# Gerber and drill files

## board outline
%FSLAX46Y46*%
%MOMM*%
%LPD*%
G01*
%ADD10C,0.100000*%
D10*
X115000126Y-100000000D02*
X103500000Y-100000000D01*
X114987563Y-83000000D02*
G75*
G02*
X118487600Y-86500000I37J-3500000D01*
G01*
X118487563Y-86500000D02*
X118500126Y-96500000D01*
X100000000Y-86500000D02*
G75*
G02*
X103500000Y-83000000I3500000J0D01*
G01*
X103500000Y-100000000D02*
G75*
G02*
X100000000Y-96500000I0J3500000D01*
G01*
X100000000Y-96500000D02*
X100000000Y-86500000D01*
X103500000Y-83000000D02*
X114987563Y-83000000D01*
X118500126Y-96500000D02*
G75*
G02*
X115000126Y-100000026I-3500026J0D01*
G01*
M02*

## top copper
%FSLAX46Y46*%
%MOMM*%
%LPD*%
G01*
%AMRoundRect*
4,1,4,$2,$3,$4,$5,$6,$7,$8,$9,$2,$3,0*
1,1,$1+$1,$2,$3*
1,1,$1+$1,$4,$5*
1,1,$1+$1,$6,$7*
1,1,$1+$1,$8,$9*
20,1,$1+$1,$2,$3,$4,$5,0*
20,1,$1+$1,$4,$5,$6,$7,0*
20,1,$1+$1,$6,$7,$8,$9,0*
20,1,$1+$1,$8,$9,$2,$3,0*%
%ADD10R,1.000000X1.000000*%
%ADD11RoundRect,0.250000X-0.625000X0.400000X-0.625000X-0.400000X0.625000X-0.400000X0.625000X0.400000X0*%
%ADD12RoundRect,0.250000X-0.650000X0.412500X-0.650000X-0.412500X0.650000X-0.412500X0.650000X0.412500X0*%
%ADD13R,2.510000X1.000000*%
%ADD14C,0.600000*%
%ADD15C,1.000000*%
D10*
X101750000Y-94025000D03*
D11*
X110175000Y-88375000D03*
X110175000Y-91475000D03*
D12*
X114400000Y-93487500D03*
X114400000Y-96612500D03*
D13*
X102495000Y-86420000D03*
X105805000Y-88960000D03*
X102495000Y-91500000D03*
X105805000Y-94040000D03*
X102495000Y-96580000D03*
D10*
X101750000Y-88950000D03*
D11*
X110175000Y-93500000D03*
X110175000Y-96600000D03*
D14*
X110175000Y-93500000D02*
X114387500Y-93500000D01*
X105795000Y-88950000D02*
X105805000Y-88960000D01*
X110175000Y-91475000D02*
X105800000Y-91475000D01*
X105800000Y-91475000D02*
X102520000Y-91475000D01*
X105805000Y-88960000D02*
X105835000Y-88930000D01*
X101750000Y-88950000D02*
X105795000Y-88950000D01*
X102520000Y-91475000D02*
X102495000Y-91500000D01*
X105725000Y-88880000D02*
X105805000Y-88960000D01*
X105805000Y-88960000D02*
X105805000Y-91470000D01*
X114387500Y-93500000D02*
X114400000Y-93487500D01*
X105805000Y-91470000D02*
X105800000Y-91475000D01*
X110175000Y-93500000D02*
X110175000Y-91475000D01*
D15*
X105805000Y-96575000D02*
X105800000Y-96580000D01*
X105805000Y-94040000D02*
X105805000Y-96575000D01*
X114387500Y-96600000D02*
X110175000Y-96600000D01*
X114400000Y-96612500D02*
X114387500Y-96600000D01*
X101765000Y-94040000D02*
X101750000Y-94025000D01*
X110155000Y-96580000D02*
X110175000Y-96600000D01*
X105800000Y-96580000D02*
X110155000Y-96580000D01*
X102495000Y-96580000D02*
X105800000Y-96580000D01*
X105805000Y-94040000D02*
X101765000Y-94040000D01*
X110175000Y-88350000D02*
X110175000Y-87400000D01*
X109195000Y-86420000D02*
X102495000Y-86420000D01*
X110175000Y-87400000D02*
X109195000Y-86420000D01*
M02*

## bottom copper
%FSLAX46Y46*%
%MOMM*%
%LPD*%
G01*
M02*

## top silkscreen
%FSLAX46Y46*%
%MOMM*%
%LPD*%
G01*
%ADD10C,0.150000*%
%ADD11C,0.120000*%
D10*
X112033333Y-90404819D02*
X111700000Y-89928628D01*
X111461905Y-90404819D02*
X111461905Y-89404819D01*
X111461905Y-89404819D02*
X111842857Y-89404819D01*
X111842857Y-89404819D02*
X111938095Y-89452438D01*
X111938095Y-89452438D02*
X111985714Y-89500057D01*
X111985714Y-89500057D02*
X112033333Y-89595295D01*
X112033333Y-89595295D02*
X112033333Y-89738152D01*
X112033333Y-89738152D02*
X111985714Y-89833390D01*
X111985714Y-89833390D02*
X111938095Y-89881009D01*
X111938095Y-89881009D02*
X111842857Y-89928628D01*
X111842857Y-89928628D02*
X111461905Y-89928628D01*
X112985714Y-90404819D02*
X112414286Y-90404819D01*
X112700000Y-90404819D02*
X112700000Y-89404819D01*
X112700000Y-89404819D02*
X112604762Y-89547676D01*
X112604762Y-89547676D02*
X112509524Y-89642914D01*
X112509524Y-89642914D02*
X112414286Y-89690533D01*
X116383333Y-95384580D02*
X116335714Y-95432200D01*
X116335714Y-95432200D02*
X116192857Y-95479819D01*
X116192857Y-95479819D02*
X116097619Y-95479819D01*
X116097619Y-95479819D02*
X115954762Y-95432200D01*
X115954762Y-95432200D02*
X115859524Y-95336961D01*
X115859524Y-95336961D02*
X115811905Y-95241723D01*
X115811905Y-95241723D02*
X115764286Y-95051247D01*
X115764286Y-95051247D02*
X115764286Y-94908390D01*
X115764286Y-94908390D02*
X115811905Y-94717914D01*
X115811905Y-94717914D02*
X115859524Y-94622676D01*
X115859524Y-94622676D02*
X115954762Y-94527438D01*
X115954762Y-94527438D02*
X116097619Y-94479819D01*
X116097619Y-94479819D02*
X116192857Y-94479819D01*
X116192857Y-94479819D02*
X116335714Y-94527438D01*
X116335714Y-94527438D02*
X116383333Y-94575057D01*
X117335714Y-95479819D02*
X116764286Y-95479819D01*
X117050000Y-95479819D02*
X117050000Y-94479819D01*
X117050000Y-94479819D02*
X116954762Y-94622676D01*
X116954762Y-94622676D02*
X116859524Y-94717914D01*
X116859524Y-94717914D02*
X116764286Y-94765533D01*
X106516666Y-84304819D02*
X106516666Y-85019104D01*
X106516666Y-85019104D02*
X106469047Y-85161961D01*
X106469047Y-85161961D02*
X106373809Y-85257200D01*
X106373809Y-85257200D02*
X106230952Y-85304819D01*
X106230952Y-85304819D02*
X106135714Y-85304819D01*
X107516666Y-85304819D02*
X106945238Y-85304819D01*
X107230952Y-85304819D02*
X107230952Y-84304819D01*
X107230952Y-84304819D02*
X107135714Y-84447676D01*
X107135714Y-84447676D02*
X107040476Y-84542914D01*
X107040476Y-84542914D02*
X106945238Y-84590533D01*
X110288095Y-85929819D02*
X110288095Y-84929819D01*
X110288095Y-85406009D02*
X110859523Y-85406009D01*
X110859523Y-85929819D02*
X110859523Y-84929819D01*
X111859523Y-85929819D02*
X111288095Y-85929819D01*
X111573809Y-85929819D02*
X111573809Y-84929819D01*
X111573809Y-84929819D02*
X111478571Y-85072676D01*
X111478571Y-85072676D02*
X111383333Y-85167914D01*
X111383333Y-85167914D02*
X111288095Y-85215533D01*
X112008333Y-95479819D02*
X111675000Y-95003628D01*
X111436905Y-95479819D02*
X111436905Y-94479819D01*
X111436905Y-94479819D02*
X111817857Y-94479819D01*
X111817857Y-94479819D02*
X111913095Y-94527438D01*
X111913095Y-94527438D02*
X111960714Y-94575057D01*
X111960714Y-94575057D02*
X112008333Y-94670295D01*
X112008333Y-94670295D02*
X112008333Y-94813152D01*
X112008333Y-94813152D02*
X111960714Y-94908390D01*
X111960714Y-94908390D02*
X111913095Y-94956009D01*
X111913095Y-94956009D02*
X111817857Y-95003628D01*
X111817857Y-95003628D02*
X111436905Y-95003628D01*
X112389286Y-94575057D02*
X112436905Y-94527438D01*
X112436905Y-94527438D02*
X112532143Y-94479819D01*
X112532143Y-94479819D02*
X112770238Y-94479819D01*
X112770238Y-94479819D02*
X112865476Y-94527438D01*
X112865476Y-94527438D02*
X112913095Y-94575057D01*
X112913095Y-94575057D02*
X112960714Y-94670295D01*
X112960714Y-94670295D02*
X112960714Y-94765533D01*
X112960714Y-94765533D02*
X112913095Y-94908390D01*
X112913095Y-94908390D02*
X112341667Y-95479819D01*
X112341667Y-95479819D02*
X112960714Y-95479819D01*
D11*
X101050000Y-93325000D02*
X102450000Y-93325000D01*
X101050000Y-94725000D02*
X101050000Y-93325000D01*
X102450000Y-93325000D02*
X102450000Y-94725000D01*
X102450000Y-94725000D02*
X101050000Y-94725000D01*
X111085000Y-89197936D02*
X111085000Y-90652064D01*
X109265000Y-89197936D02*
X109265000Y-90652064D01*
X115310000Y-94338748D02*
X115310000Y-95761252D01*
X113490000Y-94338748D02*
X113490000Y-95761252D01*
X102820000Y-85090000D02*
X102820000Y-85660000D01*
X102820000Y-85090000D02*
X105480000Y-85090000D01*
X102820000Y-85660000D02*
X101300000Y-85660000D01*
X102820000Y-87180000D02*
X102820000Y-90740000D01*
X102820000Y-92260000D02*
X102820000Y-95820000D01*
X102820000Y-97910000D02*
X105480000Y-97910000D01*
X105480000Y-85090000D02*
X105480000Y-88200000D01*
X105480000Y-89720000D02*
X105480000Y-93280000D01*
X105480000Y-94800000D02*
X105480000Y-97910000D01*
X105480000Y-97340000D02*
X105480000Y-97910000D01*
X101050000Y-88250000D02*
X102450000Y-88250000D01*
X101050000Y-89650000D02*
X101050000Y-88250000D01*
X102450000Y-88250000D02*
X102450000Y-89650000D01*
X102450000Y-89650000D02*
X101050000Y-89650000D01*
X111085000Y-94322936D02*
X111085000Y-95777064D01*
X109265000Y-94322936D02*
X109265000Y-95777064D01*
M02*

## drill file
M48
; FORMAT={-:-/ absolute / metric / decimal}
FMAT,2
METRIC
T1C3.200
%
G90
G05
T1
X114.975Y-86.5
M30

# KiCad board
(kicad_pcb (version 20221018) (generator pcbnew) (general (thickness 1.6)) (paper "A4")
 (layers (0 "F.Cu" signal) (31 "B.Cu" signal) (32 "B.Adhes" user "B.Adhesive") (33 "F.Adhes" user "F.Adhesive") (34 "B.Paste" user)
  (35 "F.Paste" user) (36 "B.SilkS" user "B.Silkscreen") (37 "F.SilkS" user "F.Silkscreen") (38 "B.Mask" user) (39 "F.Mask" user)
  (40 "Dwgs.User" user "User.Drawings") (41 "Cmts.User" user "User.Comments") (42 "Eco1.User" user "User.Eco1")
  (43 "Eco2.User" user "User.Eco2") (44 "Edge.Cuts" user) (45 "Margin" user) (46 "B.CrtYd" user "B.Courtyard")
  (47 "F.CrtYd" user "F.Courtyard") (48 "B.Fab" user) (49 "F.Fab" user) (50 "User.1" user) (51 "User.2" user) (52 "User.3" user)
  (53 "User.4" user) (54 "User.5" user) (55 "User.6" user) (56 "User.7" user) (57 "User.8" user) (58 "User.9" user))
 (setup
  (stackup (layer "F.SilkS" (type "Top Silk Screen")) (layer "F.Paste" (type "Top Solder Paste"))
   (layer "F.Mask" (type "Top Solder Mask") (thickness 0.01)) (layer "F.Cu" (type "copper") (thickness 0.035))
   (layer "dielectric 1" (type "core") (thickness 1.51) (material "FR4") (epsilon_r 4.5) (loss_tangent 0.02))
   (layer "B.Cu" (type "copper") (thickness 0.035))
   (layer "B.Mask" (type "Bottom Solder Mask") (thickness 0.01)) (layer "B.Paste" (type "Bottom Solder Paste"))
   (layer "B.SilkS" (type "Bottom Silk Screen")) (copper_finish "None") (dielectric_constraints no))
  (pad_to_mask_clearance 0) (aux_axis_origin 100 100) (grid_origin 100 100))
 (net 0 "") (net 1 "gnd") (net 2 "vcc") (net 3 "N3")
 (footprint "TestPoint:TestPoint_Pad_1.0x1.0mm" (layer "F.Cu") (at 101.75 94.025)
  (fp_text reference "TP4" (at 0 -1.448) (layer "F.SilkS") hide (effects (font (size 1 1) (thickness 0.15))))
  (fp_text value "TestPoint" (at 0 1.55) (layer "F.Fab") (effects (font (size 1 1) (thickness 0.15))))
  (fp_line (start -0.7 -0.7) (end 0.7 -0.7) (stroke (width 0.12) (type solid)) (layer "F.SilkS"))
  (fp_line (start -0.7 0.7) (end -0.7 -0.7) (stroke (width 0.12) (type solid)) (layer "F.SilkS"))
  (fp_line (start 0.7 -0.7) (end 0.7 0.7) (stroke (width 0.12) (type solid)) (layer "F.SilkS"))
  (fp_line (start 0.7 0.7) (end -0.7 0.7) (stroke (width 0.12) (type solid)) (layer "F.SilkS"))
  (pad "1" smd rect (at 0 0) (size 1 1) (layers "F.Cu" "F.Mask") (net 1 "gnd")))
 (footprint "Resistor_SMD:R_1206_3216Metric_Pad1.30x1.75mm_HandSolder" (layer "F.Cu") (at 110.175 89.925 -90)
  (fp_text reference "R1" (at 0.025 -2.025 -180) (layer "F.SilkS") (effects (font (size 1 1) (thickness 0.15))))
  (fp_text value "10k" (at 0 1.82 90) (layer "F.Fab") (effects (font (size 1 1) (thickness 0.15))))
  (fp_line (start -0.727064 -0.91) (end 0.727064 -0.91) (stroke (width 0.12) (type solid)) (layer "F.SilkS"))
  (fp_line (start -0.727064 0.91) (end 0.727064 0.91) (stroke (width 0.12) (type solid)) (layer "F.SilkS"))
  (pad "1" smd roundrect (at -1.55 0 270) (size 1.3 1.75) (layers "F.Cu" "F.Paste" "F.Mask") (roundrect_rratio 0.1923076923) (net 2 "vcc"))
  (pad "2" smd roundrect (at 1.55 0 270) (size 1.3 1.75) (layers "F.Cu" "F.Paste" "F.Mask") (roundrect_rratio 0.1923076923) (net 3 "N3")))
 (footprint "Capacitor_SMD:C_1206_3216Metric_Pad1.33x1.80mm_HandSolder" (layer "F.Cu") (at 114.4 95.05 -90)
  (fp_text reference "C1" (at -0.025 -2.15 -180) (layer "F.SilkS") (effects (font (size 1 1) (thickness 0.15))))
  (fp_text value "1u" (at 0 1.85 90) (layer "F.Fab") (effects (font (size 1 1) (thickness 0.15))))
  (fp_line (start -0.711252 -0.91) (end 0.711252 -0.91) (stroke (width 0.12) (type solid)) (layer "F.SilkS"))
  (fp_line (start -0.711252 0.91) (end 0.711252 0.91) (stroke (width 0.12) (type solid)) (layer "F.SilkS"))
  (pad "1" smd roundrect (at -1.5625 0 270) (size 1.325 1.8) (layers "F.Cu" "F.Paste" "F.Mask") (roundrect_rratio 0.1886792453) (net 3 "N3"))
  (pad "2" smd roundrect (at 1.5625 0 270) (size 1.325 1.8) (layers "F.Cu" "F.Paste" "F.Mask") (roundrect_rratio 0.1886792453) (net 1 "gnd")))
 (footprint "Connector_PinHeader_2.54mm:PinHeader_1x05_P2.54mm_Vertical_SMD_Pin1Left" (layer "F.Cu") (at 104.15 91.5)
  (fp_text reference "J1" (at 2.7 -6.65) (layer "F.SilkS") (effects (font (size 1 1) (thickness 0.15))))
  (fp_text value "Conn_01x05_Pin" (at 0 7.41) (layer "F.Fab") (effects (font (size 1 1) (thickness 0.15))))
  (fp_line (start -1.33 -6.41) (end -1.33 -5.84) (stroke (width 0.12) (type solid)) (layer "F.SilkS"))
  (fp_line (start -1.33 -6.41) (end 1.33 -6.41) (stroke (width 0.12) (type solid)) (layer "F.SilkS"))
  (fp_line (start -1.33 -5.84) (end -2.85 -5.84) (stroke (width 0.12) (type solid)) (layer "F.SilkS"))
  (fp_line (start -1.33 -4.32) (end -1.33 -0.76) (stroke (width 0.12) (type solid)) (layer "F.SilkS"))
  (fp_line (start -1.33 0.76) (end -1.33 4.32) (stroke (width 0.12) (type solid)) (layer "F.SilkS"))
  (fp_line (start -1.33 6.41) (end 1.33 6.41) (stroke (width 0.12) (type solid)) (layer "F.SilkS"))
  (fp_line (start 1.33 -6.41) (end 1.33 -3.3) (stroke (width 0.12) (type solid)) (layer "F.SilkS"))
  (fp_line (start 1.33 -1.78) (end 1.33 1.78) (stroke (width 0.12) (type solid)) (layer "F.SilkS"))
  (fp_line (start 1.33 3.3) (end 1.33 6.41) (stroke (width 0.12) (type solid)) (layer "F.SilkS"))
  (fp_line (start 1.33 5.84) (end 1.33 6.41) (stroke (width 0.12) (type solid)) (layer "F.SilkS"))
  (pad "1" smd rect (at -1.655 -5.08) (size 2.51 1) (layers "F.Cu" "F.Paste" "F.Mask") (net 2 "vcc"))
  (pad "2" smd rect (at 1.655 -2.54) (size 2.51 1) (layers "F.Cu" "F.Paste" "F.Mask") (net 3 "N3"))
  (pad "3" smd rect (at -1.655 0) (size 2.51 1) (layers "F.Cu" "F.Paste" "F.Mask") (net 3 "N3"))
  (pad "4" smd rect (at 1.655 2.54) (size 2.51 1) (layers "F.Cu" "F.Paste" "F.Mask") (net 1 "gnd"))
  (pad "5" smd rect (at -1.655 5.08) (size 2.51 1) (layers "F.Cu" "F.Paste" "F.Mask") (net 1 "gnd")))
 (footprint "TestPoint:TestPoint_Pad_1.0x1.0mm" (layer "F.Cu") (at 101.75 88.95)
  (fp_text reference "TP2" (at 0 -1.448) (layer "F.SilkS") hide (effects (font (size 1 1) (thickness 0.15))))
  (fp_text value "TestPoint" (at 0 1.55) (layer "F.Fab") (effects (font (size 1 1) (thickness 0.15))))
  (fp_line (start -0.7 -0.7) (end 0.7 -0.7) (stroke (width 0.12) (type solid)) (layer "F.SilkS"))
  (fp_line (start -0.7 0.7) (end -0.7 -0.7) (stroke (width 0.12) (type solid)) (layer "F.SilkS"))
  (fp_line (start 0.7 -0.7) (end 0.7 0.7) (stroke (width 0.12) (type solid)) (layer "F.SilkS"))
  (fp_line (start 0.7 0.7) (end -0.7 0.7) (stroke (width 0.12) (type solid)) (layer "F.SilkS"))
  (pad "1" smd rect (at 0 0) (size 1 1) (layers "F.Cu" "F.Mask") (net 3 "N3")))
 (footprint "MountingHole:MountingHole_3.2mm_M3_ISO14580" (layer "F.Cu") (at 114.975 86.5)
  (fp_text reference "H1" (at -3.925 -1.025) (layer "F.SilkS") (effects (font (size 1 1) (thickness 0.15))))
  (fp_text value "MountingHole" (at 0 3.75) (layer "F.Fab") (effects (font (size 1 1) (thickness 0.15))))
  (pad "" np_thru_hole circle (at 0 0) (size 3.2 3.2) (drill 3.2) (layers "*.Cu" "*.Mask")))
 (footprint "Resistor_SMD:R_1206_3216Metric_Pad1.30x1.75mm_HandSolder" (layer "F.Cu") (at 110.175 95.05 -90)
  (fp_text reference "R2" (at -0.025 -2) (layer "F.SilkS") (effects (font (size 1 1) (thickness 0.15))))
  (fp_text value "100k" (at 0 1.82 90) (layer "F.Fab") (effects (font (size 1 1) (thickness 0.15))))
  (fp_line (start -0.727064 -0.91) (end 0.727064 -0.91) (stroke (width 0.12) (type solid)) (layer "F.SilkS"))
  (fp_line (start -0.727064 0.91) (end 0.727064 0.91) (stroke (width 0.12) (type solid)) (layer "F.SilkS"))
  (pad "1" smd roundrect (at -1.55 0 270) (size 1.3 1.75) (layers "F.Cu" "F.Paste" "F.Mask") (roundrect_rratio 0.1923076923) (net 3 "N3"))
  (pad "2" smd roundrect (at 1.55 0 270) (size 1.3 1.75) (layers "F.Cu" "F.Paste" "F.Mask") (roundrect_rratio 0.1923076923) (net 1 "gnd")))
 (gr_line (start 115.000126 100) (end 103.5 100) (stroke (width 0.1) (type default)) (layer "Edge.Cuts"))
 (gr_arc (start 114.987563 83) (mid 117.462436 84.025126) (end 118.487563 86.5) (stroke (width 0.1) (type default)) (layer "Edge.Cuts"))
 (gr_line (start 118.487563 86.5) (end 118.500126 96.5) (stroke (width 0.1) (type default)) (layer "Edge.Cuts"))
 (gr_arc (start 100 86.5) (mid 101.025126 84.025126) (end 103.5 83) (stroke (width 0.1) (type default)) (layer "Edge.Cuts"))
 (gr_arc (start 103.5 100) (mid 101.025126 98.974874) (end 100 96.5) (stroke (width 0.1) (type default)) (layer "Edge.Cuts"))
 (gr_line (start 100 96.5) (end 100 86.5) (stroke (width 0.1) (type default)) (layer "Edge.Cuts"))
 (gr_line (start 103.5 83) (end 114.987563 83) (stroke (width 0.1) (type default)) (layer "Edge.Cuts"))
 (gr_arc (start 118.500126 96.5) (mid 117.475 98.974874) (end 115.000126 100) (stroke (width 0.1) (type default)) (layer "Edge.Cuts"))
 (segment (start 110.175 93.5) (end 114.3875 93.5) (width 0.6) (layer "F.Cu") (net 3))
 (segment (start 105.795 88.95) (end 105.805 88.96) (width 0.6) (layer "F.Cu") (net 3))
 (segment (start 110.175 91.475) (end 105.8 91.475) (width 0.6) (layer "F.Cu") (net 3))
 (segment (start 105.8 91.475) (end 102.52 91.475) (width 0.6) (layer "F.Cu") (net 3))
 (segment (start 105.805 88.96) (end 105.835 88.93) (width 0.6) (layer "F.Cu") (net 3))
 (segment (start 101.75 88.95) (end 105.795 88.95) (width 0.6) (layer "F.Cu") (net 3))
 (segment (start 102.52 91.475) (end 102.495 91.5) (width 0.6) (layer "F.Cu") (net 3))
 (segment (start 105.725 88.88) (end 105.805 88.96) (width 0.6) (layer "F.Cu") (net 3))
 (segment (start 105.805 88.96) (end 105.805 91.47) (width 0.6) (layer "F.Cu") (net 3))
 (segment (start 114.3875 93.5) (end 114.4 93.4875) (width 0.6) (layer "F.Cu") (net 3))
 (segment (start 105.805 91.47) (end 105.8 91.475) (width 0.6) (layer "F.Cu") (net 3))
 (segment (start 110.175 93.5) (end 110.175 91.475) (width 0.6) (layer "F.Cu") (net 3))
 (segment (start 105.805 96.575) (end 105.8 96.58) (width 1) (layer "F.Cu") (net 1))
 (segment (start 105.805 94.04) (end 105.805 96.575) (width 1) (layer "F.Cu") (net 1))
 (segment (start 114.3875 96.6) (end 110.175 96.6) (width 1) (layer "F.Cu") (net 1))
 (segment (start 114.4 96.6125) (end 114.3875 96.6) (width 1) (layer "F.Cu") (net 1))
 (segment (start 101.765 94.04) (end 101.75 94.025) (width 1) (layer "F.Cu") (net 1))
 (segment (start 110.155 96.58) (end 110.175 96.6) (width 1) (layer "F.Cu") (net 1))
 (segment (start 105.8 96.58) (end 110.155 96.58) (width 1) (layer "F.Cu") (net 1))
 (segment (start 102.495 96.58) (end 105.8 96.58) (width 1) (layer "F.Cu") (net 1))
 (segment (start 105.805 94.04) (end 101.765 94.04) (width 1) (layer "F.Cu") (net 1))
 (segment (start 110.175 88.35) (end 110.175 87.4) (width 1) (layer "F.Cu") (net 2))
 (segment (start 109.195 86.42) (end 102.495 86.42) (width 1) (layer "F.Cu") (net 2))
 (segment (start 110.175 87.4) (end 109.195 86.42) (width 1) (layer "F.Cu") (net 2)))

